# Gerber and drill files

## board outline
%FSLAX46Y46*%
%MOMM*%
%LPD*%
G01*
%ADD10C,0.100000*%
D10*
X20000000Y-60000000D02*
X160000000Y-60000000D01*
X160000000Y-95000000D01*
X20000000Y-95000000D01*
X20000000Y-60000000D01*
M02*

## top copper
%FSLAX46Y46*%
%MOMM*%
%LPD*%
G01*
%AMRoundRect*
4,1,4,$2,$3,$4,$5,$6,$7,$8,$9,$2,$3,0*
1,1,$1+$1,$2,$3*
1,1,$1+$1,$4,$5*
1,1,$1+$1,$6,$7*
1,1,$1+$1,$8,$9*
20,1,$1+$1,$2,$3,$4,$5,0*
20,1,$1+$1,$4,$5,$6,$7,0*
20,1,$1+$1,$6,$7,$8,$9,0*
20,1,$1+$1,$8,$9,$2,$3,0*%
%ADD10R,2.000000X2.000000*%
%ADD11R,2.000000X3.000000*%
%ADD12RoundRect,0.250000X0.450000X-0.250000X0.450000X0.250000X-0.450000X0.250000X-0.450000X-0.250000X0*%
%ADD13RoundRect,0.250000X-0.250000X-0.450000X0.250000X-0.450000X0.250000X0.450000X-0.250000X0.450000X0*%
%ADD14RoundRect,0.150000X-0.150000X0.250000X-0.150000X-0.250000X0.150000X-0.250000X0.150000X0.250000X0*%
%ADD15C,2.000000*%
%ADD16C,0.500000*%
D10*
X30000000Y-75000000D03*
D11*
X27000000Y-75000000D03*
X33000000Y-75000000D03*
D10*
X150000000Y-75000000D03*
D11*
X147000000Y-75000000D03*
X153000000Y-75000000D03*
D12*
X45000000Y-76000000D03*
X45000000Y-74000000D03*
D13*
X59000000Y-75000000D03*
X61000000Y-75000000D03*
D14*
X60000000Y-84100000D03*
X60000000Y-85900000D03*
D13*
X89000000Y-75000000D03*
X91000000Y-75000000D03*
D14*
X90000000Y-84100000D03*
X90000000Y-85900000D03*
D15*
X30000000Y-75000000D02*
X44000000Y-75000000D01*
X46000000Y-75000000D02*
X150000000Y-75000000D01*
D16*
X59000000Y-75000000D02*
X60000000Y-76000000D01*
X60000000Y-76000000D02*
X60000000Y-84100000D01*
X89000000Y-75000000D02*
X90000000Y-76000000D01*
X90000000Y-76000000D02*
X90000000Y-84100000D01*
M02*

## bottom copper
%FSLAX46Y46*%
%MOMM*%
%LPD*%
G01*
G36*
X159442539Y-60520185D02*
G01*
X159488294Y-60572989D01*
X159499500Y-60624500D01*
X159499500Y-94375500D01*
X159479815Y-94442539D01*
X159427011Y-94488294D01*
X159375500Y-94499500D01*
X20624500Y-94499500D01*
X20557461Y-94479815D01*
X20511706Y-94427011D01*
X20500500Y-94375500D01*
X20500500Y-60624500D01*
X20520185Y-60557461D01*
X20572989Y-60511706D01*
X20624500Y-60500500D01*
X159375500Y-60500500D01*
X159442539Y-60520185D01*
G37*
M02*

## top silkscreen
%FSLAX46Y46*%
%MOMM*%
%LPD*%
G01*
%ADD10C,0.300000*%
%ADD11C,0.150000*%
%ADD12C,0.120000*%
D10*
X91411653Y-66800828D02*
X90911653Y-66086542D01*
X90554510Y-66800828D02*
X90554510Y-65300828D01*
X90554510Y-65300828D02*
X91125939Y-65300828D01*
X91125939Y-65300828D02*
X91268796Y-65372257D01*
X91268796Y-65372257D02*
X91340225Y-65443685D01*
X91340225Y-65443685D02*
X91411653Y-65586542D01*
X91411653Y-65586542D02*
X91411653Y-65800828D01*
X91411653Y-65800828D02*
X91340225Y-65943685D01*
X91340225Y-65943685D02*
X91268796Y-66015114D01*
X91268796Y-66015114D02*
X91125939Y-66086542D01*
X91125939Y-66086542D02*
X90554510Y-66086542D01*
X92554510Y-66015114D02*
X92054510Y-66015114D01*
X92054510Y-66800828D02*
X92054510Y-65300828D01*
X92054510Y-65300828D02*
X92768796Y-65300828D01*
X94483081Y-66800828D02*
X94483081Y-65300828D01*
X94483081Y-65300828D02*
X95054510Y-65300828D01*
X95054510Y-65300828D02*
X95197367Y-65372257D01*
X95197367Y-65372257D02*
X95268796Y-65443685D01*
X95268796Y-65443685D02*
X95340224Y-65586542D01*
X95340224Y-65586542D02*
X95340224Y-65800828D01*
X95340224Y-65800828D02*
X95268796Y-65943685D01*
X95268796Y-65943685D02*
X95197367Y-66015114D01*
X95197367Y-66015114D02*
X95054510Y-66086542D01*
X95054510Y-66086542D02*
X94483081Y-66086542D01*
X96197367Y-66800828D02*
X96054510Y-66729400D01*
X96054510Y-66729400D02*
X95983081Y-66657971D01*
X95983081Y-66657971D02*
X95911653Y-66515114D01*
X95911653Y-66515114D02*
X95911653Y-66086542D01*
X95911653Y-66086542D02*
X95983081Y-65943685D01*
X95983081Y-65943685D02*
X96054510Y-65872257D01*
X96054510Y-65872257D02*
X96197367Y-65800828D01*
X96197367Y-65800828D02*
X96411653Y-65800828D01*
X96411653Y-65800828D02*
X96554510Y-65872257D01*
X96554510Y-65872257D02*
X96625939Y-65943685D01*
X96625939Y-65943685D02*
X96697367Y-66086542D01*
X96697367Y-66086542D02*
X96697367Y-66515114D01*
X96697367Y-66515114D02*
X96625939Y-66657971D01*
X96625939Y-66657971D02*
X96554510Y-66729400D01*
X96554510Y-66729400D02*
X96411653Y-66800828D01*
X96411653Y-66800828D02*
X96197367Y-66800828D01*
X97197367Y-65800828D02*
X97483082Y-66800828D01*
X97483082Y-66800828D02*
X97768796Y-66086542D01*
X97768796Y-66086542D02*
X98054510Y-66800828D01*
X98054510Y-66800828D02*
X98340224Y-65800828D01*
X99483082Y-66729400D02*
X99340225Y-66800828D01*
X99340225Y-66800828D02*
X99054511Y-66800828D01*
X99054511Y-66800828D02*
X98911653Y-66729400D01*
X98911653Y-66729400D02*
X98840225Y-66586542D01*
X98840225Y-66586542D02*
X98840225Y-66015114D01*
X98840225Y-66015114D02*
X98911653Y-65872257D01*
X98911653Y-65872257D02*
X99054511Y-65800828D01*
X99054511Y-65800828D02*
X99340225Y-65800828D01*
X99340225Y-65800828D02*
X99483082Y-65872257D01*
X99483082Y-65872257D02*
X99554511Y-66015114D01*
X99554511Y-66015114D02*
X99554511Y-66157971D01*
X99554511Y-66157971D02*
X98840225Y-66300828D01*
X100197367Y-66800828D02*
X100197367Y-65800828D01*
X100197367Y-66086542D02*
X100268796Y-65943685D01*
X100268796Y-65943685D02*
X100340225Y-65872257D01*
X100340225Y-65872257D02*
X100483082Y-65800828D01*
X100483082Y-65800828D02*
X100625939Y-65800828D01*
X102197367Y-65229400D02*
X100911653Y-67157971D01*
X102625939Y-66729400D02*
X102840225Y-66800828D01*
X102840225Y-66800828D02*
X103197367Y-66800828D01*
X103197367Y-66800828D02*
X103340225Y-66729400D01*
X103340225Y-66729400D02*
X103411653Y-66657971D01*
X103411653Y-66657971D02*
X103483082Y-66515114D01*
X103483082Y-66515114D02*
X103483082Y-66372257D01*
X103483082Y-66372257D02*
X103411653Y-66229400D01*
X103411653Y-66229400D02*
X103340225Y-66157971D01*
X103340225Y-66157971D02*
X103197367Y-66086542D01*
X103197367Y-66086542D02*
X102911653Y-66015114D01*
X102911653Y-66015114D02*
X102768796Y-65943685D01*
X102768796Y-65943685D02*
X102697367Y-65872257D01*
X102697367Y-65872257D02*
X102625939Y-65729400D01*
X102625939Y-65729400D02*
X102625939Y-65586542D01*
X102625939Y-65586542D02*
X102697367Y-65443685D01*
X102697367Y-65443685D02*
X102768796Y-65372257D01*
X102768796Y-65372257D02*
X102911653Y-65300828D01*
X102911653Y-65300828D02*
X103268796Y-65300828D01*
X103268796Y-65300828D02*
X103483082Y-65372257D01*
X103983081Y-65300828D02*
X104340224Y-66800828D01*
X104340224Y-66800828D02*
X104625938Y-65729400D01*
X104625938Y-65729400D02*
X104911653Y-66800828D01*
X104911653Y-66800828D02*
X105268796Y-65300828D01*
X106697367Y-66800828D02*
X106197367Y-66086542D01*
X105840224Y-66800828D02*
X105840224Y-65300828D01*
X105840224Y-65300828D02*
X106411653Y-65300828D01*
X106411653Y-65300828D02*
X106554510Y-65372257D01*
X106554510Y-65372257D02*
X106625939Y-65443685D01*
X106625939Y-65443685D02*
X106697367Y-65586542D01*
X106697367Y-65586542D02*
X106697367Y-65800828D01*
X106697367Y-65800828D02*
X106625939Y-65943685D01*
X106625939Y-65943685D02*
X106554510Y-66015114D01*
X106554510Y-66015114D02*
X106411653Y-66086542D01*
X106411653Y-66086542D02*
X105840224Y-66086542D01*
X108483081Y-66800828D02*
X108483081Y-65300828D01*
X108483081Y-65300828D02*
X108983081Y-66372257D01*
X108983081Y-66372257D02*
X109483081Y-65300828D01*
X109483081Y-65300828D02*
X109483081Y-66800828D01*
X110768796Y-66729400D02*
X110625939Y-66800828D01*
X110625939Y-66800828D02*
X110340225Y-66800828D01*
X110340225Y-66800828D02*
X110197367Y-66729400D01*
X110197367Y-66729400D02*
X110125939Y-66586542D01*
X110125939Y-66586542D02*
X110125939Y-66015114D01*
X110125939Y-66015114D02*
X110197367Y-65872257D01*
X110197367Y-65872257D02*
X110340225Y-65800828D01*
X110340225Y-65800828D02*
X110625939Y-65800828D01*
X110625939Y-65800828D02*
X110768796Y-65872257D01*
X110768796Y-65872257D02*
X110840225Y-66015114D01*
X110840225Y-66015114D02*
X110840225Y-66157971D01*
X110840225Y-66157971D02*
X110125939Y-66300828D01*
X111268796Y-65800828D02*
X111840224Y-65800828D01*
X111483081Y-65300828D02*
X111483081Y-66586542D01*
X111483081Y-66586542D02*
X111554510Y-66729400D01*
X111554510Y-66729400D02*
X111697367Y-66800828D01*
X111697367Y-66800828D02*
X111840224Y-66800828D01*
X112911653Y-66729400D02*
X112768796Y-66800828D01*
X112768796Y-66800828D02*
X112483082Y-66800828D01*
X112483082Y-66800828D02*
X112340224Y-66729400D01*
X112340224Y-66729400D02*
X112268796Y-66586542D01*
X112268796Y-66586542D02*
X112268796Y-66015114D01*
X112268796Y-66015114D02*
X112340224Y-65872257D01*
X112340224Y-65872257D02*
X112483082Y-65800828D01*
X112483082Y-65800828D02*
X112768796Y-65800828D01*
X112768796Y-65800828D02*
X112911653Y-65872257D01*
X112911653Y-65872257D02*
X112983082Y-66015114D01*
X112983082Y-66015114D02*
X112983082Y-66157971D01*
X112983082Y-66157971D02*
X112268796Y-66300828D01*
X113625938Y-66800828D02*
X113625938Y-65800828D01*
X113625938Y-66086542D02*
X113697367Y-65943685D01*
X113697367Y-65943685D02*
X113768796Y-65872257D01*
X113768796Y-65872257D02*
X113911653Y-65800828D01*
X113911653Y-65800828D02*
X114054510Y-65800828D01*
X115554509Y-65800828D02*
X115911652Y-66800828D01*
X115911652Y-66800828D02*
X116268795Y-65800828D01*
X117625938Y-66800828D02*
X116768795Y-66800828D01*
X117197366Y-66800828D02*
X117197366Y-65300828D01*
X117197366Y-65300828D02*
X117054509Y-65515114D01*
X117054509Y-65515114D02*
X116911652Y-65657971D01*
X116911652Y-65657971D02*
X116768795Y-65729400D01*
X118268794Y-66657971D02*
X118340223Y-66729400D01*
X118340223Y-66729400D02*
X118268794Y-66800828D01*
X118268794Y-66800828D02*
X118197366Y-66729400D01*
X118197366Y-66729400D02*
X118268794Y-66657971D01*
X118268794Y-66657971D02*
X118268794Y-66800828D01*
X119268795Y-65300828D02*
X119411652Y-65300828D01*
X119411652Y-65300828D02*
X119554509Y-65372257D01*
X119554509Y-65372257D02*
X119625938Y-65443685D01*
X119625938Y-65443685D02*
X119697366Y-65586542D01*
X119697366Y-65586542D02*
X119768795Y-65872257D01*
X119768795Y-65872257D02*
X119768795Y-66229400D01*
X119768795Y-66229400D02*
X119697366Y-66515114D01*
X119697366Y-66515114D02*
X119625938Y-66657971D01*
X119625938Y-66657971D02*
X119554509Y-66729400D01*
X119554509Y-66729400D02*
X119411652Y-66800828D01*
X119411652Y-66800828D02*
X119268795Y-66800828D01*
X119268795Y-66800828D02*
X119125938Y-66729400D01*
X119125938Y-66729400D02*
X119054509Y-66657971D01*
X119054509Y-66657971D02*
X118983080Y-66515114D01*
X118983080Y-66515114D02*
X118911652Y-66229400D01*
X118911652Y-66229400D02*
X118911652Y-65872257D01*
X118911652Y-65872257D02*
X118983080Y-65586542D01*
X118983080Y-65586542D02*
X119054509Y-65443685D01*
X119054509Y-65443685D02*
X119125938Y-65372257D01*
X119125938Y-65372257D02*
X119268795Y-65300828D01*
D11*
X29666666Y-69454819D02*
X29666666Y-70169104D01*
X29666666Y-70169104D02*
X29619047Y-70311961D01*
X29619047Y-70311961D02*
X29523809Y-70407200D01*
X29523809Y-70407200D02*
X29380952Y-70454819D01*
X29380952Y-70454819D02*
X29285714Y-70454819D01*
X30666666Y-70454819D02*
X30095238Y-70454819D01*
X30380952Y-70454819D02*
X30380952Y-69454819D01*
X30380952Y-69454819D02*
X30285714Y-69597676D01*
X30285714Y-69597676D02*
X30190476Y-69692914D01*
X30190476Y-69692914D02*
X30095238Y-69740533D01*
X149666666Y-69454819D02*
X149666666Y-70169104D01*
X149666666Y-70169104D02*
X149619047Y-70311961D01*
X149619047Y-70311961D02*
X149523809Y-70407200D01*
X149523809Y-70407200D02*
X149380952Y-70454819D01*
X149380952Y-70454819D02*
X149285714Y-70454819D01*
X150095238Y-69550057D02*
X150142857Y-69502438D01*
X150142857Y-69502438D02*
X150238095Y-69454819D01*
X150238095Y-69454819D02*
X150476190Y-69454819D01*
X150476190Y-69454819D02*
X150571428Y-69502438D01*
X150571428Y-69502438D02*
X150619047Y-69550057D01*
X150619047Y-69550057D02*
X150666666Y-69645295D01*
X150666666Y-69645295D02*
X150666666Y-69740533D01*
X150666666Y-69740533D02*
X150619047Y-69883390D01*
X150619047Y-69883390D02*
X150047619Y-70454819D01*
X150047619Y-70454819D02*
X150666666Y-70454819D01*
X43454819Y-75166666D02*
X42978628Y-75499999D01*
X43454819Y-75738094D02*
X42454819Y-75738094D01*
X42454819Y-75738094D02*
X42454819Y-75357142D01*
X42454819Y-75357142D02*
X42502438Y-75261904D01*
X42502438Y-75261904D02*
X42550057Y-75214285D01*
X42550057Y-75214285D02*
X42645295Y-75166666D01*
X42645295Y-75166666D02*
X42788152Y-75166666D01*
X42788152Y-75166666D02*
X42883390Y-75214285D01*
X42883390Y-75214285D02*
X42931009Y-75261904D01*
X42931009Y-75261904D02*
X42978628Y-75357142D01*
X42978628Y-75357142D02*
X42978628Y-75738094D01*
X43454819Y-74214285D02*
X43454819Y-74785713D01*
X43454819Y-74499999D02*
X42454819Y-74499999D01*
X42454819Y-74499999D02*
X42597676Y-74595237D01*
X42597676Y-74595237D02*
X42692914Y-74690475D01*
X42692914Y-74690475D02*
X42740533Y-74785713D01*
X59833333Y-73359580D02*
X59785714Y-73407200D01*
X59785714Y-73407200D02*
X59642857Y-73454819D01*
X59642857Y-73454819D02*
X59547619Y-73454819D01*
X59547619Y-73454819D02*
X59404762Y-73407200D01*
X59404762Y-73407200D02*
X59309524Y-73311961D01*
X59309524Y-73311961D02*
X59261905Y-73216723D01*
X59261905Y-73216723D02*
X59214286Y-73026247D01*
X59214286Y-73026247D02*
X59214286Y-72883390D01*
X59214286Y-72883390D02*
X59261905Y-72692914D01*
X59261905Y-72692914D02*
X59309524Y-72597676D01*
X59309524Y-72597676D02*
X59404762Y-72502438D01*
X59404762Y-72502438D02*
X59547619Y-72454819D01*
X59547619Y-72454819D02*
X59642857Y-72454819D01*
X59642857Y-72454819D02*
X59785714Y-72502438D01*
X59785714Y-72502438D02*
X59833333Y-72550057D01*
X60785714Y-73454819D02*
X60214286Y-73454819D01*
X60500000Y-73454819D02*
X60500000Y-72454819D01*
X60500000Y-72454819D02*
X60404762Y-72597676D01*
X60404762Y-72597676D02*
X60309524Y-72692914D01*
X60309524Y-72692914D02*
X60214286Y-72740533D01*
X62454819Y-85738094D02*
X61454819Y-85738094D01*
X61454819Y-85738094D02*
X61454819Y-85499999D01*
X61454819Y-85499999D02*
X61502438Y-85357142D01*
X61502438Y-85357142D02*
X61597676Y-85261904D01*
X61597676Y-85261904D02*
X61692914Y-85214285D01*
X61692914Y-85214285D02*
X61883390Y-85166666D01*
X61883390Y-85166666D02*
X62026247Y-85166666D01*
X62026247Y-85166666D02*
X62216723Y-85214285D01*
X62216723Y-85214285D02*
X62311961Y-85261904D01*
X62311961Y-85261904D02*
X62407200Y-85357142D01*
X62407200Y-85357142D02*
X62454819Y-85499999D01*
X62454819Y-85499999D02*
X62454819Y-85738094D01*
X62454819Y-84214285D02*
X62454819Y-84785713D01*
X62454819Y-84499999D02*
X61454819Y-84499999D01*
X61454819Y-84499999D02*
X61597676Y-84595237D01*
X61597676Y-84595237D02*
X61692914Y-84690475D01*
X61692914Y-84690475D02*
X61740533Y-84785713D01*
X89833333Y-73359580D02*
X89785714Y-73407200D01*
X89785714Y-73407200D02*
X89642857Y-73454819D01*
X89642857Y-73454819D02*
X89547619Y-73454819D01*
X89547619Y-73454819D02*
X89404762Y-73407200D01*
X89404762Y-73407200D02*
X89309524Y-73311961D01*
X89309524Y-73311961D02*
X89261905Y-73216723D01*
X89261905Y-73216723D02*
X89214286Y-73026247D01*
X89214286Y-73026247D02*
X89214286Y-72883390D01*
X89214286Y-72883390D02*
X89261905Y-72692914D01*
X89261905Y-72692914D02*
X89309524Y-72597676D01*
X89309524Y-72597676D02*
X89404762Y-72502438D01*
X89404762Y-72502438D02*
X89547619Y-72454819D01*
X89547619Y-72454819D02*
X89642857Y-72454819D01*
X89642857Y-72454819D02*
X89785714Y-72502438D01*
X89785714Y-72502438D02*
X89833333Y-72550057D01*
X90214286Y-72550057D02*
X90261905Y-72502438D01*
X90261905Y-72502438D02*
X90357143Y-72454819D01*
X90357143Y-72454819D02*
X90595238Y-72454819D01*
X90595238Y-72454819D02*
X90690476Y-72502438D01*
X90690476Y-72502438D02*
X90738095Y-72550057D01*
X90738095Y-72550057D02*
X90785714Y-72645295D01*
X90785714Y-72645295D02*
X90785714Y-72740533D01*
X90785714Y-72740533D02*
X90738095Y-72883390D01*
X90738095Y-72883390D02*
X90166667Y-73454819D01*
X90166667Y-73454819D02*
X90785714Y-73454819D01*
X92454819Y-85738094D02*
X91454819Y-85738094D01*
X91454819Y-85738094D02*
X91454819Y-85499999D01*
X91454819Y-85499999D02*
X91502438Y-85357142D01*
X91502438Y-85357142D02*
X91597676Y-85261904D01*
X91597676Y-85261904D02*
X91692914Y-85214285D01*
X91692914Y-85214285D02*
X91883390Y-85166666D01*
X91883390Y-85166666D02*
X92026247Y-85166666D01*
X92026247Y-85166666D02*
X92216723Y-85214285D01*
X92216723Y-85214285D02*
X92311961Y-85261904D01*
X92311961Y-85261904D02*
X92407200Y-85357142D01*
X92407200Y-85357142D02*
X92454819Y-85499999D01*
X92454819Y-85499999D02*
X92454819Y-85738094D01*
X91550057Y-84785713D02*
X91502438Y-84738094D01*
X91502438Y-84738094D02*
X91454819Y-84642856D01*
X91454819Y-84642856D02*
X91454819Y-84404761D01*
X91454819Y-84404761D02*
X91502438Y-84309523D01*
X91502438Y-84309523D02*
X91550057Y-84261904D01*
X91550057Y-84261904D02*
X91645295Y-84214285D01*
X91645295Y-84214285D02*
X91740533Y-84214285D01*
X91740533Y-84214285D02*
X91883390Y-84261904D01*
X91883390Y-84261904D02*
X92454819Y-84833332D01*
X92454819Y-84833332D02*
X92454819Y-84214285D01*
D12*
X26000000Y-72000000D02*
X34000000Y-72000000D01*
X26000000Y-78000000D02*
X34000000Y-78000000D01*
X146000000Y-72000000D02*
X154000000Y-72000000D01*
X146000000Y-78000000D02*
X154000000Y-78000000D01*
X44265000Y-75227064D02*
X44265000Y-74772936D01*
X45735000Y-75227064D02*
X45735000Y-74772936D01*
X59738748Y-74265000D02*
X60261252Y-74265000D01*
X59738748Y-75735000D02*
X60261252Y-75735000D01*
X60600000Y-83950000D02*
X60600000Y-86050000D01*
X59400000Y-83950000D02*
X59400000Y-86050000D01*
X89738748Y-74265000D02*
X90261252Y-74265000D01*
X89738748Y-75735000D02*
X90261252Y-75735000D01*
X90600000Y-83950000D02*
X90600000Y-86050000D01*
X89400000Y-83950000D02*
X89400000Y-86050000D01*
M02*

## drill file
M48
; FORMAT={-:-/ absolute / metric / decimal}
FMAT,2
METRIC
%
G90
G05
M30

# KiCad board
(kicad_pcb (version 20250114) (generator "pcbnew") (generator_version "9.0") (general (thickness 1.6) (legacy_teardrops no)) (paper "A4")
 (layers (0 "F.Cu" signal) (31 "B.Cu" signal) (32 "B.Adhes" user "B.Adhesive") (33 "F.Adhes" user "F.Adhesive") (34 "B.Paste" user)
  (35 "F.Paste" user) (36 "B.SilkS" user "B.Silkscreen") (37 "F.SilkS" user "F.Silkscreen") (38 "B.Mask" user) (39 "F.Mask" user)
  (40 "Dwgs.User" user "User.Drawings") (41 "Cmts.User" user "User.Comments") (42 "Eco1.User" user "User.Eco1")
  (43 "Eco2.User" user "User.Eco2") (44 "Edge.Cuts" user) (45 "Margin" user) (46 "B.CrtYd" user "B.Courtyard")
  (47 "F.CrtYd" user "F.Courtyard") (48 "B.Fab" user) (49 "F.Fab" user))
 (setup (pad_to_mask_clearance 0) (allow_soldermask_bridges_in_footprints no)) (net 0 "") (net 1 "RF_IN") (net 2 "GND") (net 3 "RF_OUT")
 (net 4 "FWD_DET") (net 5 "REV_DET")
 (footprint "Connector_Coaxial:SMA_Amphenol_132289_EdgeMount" (layer "F.Cu") (at 30 75 0)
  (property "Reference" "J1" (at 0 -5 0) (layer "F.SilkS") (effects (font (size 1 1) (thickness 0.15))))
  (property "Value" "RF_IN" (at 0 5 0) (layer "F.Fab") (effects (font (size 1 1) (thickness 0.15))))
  (fp_line (start -4 -3) (end 4 -3) (stroke (width 0.12) (type solid)) (layer "F.SilkS"))
  (fp_line (start -4 3) (end 4 3) (stroke (width 0.12) (type solid)) (layer "F.SilkS"))
  (pad "1" smd rect (at 0 0) (size 2 2) (layers "F.Cu" "F.Paste" "F.Mask") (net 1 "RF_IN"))
  (pad "2" smd rect (at -3 0) (size 2 3) (layers "F.Cu" "F.Paste" "F.Mask") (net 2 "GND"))
  (pad "2" smd rect (at 3 0) (size 2 3) (layers "F.Cu" "F.Paste" "F.Mask") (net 2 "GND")))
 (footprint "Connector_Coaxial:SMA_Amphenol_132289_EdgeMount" (layer "F.Cu") (at 150 75 0)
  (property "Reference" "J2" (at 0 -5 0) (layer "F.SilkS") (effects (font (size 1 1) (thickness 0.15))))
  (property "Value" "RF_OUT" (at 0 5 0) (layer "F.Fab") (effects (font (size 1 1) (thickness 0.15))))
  (fp_line (start -4 -3) (end 4 -3) (stroke (width 0.12) (type solid)) (layer "F.SilkS"))
  (fp_line (start -4 3) (end 4 3) (stroke (width 0.12) (type solid)) (layer "F.SilkS"))
  (pad "1" smd rect (at 0 0) (size 2 2) (layers "F.Cu" "F.Paste" "F.Mask") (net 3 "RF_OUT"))
  (pad "2" smd rect (at -3 0) (size 2 3) (layers "F.Cu" "F.Paste" "F.Mask") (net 2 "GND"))
  (pad "2" smd rect (at 3 0) (size 2 3) (layers "F.Cu" "F.Paste" "F.Mask") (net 2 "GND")))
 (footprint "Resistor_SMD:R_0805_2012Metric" (layer "F.Cu") (at 45 75 90)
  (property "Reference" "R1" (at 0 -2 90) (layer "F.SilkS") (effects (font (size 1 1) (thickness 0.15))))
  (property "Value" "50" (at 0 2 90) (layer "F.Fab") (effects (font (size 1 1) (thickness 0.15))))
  (fp_line (start -0.227064 -0.735) (end 0.227064 -0.735) (stroke (width 0.12) (type solid)) (layer "F.SilkS"))
  (fp_line (start -0.227064 0.735) (end 0.227064 0.735) (stroke (width 0.12) (type solid)) (layer "F.SilkS"))
  (pad "1" smd roundrect (at -1 0 90) (size 1 1.4) (layers "F.Cu" "F.Paste" "F.Mask") (roundrect_rratio 0.25) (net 1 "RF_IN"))
  (pad "2" smd roundrect (at 1 0 90) (size 1 1.4) (layers "F.Cu" "F.Paste" "F.Mask") (roundrect_rratio 0.25) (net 2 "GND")))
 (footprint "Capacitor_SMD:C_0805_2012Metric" (layer "F.Cu") (at 60 75 0)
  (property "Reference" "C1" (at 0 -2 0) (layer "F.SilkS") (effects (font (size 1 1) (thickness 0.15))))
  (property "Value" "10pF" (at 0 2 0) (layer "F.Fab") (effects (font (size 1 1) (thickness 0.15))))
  (fp_line (start -0.261252 -0.735) (end 0.261252 -0.735) (stroke (width 0.12) (type solid)) (layer "F.SilkS"))
  (fp_line (start -0.261252 0.735) (end 0.261252 0.735) (stroke (width 0.12) (type solid)) (layer "F.SilkS"))
  (pad "1" smd roundrect (at -1 0) (size 1 1.4) (layers "F.Cu" "F.Paste" "F.Mask") (roundrect_rratio 0.25) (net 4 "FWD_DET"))
  (pad "2" smd roundrect (at 1 0) (size 1 1.4) (layers "F.Cu" "F.Paste" "F.Mask") (roundrect_rratio 0.25) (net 2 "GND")))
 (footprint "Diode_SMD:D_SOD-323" (layer "F.Cu") (at 60 85 270)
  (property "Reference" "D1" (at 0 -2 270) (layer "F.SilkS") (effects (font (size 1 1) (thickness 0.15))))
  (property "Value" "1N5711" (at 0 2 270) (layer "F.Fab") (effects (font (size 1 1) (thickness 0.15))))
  (fp_line (start -1.05 -0.6) (end 1.05 -0.6) (stroke (width 0.12) (type solid)) (layer "F.SilkS"))
  (fp_line (start -1.05 0.6) (end 1.05 0.6) (stroke (width 0.12) (type solid)) (layer "F.SilkS"))
  (pad "1" smd roundrect (at -0.9 0 270) (size 0.8 0.6) (layers "F.Cu" "F.Paste" "F.Mask") (roundrect_rratio 0.25) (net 4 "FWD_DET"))
  (pad "2" smd roundrect (at 0.9 0 270) (size 0.8 0.6) (layers "F.Cu" "F.Paste" "F.Mask") (roundrect_rratio 0.25) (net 2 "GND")))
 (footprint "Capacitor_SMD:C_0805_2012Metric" (layer "F.Cu") (at 90 75 0)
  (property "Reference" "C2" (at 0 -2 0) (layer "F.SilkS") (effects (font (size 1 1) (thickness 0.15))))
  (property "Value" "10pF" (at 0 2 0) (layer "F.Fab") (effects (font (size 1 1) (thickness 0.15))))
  (fp_line (start -0.261252 -0.735) (end 0.261252 -0.735) (stroke (width 0.12) (type solid)) (layer "F.SilkS"))
  (fp_line (start -0.261252 0.735) (end 0.261252 0.735) (stroke (width 0.12) (type solid)) (layer "F.SilkS"))
  (pad "1" smd roundrect (at -1 0) (size 1 1.4) (layers "F.Cu" "F.Paste" "F.Mask") (roundrect_rratio 0.25) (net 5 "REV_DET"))
  (pad "2" smd roundrect (at 1 0) (size 1 1.4) (layers "F.Cu" "F.Paste" "F.Mask") (roundrect_rratio 0.25) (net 2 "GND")))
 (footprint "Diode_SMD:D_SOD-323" (layer "F.Cu") (at 90 85 270)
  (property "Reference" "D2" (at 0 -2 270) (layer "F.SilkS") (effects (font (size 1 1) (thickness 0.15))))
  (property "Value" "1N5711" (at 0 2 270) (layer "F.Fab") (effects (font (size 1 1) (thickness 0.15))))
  (fp_line (start -1.05 -0.6) (end 1.05 -0.6) (stroke (width 0.12) (type solid)) (layer "F.SilkS"))
  (fp_line (start -1.05 0.6) (end 1.05 0.6) (stroke (width 0.12) (type solid)) (layer "F.SilkS"))
  (pad "1" smd roundrect (at -0.9 0 270) (size 0.8 0.6) (layers "F.Cu" "F.Paste" "F.Mask") (roundrect_rratio 0.25) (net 5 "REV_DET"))
  (pad "2" smd roundrect (at 0.9 0 270) (size 0.8 0.6) (layers "F.Cu" "F.Paste" "F.Mask") (roundrect_rratio 0.25) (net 2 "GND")))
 (gr_rect (start 20 60) (end 160 95) (stroke (width 0.1) (type default)) (fill none) (layer "Edge.Cuts"))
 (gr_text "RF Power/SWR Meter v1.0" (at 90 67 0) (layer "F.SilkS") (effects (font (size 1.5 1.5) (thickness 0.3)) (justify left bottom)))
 (segment (start 30 75) (end 44 75) (width 2) (layer "F.Cu") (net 1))
 (segment (start 46 75) (end 150 75) (width 2) (layer "F.Cu") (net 3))
 (segment (start 59 75) (end 60 76) (width 0.5) (layer "F.Cu") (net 4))
 (segment (start 60 76) (end 60 84.1) (width 0.5) (layer "F.Cu") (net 4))
 (segment (start 89 75) (end 90 76) (width 0.5) (layer "F.Cu") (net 5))
 (segment (start 90 76) (end 90 84.1) (width 0.5) (layer "F.Cu") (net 5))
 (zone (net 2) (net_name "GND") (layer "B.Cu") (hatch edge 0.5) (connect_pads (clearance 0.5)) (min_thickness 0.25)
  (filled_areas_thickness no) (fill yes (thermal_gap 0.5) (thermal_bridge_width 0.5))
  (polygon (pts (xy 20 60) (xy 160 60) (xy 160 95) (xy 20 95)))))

